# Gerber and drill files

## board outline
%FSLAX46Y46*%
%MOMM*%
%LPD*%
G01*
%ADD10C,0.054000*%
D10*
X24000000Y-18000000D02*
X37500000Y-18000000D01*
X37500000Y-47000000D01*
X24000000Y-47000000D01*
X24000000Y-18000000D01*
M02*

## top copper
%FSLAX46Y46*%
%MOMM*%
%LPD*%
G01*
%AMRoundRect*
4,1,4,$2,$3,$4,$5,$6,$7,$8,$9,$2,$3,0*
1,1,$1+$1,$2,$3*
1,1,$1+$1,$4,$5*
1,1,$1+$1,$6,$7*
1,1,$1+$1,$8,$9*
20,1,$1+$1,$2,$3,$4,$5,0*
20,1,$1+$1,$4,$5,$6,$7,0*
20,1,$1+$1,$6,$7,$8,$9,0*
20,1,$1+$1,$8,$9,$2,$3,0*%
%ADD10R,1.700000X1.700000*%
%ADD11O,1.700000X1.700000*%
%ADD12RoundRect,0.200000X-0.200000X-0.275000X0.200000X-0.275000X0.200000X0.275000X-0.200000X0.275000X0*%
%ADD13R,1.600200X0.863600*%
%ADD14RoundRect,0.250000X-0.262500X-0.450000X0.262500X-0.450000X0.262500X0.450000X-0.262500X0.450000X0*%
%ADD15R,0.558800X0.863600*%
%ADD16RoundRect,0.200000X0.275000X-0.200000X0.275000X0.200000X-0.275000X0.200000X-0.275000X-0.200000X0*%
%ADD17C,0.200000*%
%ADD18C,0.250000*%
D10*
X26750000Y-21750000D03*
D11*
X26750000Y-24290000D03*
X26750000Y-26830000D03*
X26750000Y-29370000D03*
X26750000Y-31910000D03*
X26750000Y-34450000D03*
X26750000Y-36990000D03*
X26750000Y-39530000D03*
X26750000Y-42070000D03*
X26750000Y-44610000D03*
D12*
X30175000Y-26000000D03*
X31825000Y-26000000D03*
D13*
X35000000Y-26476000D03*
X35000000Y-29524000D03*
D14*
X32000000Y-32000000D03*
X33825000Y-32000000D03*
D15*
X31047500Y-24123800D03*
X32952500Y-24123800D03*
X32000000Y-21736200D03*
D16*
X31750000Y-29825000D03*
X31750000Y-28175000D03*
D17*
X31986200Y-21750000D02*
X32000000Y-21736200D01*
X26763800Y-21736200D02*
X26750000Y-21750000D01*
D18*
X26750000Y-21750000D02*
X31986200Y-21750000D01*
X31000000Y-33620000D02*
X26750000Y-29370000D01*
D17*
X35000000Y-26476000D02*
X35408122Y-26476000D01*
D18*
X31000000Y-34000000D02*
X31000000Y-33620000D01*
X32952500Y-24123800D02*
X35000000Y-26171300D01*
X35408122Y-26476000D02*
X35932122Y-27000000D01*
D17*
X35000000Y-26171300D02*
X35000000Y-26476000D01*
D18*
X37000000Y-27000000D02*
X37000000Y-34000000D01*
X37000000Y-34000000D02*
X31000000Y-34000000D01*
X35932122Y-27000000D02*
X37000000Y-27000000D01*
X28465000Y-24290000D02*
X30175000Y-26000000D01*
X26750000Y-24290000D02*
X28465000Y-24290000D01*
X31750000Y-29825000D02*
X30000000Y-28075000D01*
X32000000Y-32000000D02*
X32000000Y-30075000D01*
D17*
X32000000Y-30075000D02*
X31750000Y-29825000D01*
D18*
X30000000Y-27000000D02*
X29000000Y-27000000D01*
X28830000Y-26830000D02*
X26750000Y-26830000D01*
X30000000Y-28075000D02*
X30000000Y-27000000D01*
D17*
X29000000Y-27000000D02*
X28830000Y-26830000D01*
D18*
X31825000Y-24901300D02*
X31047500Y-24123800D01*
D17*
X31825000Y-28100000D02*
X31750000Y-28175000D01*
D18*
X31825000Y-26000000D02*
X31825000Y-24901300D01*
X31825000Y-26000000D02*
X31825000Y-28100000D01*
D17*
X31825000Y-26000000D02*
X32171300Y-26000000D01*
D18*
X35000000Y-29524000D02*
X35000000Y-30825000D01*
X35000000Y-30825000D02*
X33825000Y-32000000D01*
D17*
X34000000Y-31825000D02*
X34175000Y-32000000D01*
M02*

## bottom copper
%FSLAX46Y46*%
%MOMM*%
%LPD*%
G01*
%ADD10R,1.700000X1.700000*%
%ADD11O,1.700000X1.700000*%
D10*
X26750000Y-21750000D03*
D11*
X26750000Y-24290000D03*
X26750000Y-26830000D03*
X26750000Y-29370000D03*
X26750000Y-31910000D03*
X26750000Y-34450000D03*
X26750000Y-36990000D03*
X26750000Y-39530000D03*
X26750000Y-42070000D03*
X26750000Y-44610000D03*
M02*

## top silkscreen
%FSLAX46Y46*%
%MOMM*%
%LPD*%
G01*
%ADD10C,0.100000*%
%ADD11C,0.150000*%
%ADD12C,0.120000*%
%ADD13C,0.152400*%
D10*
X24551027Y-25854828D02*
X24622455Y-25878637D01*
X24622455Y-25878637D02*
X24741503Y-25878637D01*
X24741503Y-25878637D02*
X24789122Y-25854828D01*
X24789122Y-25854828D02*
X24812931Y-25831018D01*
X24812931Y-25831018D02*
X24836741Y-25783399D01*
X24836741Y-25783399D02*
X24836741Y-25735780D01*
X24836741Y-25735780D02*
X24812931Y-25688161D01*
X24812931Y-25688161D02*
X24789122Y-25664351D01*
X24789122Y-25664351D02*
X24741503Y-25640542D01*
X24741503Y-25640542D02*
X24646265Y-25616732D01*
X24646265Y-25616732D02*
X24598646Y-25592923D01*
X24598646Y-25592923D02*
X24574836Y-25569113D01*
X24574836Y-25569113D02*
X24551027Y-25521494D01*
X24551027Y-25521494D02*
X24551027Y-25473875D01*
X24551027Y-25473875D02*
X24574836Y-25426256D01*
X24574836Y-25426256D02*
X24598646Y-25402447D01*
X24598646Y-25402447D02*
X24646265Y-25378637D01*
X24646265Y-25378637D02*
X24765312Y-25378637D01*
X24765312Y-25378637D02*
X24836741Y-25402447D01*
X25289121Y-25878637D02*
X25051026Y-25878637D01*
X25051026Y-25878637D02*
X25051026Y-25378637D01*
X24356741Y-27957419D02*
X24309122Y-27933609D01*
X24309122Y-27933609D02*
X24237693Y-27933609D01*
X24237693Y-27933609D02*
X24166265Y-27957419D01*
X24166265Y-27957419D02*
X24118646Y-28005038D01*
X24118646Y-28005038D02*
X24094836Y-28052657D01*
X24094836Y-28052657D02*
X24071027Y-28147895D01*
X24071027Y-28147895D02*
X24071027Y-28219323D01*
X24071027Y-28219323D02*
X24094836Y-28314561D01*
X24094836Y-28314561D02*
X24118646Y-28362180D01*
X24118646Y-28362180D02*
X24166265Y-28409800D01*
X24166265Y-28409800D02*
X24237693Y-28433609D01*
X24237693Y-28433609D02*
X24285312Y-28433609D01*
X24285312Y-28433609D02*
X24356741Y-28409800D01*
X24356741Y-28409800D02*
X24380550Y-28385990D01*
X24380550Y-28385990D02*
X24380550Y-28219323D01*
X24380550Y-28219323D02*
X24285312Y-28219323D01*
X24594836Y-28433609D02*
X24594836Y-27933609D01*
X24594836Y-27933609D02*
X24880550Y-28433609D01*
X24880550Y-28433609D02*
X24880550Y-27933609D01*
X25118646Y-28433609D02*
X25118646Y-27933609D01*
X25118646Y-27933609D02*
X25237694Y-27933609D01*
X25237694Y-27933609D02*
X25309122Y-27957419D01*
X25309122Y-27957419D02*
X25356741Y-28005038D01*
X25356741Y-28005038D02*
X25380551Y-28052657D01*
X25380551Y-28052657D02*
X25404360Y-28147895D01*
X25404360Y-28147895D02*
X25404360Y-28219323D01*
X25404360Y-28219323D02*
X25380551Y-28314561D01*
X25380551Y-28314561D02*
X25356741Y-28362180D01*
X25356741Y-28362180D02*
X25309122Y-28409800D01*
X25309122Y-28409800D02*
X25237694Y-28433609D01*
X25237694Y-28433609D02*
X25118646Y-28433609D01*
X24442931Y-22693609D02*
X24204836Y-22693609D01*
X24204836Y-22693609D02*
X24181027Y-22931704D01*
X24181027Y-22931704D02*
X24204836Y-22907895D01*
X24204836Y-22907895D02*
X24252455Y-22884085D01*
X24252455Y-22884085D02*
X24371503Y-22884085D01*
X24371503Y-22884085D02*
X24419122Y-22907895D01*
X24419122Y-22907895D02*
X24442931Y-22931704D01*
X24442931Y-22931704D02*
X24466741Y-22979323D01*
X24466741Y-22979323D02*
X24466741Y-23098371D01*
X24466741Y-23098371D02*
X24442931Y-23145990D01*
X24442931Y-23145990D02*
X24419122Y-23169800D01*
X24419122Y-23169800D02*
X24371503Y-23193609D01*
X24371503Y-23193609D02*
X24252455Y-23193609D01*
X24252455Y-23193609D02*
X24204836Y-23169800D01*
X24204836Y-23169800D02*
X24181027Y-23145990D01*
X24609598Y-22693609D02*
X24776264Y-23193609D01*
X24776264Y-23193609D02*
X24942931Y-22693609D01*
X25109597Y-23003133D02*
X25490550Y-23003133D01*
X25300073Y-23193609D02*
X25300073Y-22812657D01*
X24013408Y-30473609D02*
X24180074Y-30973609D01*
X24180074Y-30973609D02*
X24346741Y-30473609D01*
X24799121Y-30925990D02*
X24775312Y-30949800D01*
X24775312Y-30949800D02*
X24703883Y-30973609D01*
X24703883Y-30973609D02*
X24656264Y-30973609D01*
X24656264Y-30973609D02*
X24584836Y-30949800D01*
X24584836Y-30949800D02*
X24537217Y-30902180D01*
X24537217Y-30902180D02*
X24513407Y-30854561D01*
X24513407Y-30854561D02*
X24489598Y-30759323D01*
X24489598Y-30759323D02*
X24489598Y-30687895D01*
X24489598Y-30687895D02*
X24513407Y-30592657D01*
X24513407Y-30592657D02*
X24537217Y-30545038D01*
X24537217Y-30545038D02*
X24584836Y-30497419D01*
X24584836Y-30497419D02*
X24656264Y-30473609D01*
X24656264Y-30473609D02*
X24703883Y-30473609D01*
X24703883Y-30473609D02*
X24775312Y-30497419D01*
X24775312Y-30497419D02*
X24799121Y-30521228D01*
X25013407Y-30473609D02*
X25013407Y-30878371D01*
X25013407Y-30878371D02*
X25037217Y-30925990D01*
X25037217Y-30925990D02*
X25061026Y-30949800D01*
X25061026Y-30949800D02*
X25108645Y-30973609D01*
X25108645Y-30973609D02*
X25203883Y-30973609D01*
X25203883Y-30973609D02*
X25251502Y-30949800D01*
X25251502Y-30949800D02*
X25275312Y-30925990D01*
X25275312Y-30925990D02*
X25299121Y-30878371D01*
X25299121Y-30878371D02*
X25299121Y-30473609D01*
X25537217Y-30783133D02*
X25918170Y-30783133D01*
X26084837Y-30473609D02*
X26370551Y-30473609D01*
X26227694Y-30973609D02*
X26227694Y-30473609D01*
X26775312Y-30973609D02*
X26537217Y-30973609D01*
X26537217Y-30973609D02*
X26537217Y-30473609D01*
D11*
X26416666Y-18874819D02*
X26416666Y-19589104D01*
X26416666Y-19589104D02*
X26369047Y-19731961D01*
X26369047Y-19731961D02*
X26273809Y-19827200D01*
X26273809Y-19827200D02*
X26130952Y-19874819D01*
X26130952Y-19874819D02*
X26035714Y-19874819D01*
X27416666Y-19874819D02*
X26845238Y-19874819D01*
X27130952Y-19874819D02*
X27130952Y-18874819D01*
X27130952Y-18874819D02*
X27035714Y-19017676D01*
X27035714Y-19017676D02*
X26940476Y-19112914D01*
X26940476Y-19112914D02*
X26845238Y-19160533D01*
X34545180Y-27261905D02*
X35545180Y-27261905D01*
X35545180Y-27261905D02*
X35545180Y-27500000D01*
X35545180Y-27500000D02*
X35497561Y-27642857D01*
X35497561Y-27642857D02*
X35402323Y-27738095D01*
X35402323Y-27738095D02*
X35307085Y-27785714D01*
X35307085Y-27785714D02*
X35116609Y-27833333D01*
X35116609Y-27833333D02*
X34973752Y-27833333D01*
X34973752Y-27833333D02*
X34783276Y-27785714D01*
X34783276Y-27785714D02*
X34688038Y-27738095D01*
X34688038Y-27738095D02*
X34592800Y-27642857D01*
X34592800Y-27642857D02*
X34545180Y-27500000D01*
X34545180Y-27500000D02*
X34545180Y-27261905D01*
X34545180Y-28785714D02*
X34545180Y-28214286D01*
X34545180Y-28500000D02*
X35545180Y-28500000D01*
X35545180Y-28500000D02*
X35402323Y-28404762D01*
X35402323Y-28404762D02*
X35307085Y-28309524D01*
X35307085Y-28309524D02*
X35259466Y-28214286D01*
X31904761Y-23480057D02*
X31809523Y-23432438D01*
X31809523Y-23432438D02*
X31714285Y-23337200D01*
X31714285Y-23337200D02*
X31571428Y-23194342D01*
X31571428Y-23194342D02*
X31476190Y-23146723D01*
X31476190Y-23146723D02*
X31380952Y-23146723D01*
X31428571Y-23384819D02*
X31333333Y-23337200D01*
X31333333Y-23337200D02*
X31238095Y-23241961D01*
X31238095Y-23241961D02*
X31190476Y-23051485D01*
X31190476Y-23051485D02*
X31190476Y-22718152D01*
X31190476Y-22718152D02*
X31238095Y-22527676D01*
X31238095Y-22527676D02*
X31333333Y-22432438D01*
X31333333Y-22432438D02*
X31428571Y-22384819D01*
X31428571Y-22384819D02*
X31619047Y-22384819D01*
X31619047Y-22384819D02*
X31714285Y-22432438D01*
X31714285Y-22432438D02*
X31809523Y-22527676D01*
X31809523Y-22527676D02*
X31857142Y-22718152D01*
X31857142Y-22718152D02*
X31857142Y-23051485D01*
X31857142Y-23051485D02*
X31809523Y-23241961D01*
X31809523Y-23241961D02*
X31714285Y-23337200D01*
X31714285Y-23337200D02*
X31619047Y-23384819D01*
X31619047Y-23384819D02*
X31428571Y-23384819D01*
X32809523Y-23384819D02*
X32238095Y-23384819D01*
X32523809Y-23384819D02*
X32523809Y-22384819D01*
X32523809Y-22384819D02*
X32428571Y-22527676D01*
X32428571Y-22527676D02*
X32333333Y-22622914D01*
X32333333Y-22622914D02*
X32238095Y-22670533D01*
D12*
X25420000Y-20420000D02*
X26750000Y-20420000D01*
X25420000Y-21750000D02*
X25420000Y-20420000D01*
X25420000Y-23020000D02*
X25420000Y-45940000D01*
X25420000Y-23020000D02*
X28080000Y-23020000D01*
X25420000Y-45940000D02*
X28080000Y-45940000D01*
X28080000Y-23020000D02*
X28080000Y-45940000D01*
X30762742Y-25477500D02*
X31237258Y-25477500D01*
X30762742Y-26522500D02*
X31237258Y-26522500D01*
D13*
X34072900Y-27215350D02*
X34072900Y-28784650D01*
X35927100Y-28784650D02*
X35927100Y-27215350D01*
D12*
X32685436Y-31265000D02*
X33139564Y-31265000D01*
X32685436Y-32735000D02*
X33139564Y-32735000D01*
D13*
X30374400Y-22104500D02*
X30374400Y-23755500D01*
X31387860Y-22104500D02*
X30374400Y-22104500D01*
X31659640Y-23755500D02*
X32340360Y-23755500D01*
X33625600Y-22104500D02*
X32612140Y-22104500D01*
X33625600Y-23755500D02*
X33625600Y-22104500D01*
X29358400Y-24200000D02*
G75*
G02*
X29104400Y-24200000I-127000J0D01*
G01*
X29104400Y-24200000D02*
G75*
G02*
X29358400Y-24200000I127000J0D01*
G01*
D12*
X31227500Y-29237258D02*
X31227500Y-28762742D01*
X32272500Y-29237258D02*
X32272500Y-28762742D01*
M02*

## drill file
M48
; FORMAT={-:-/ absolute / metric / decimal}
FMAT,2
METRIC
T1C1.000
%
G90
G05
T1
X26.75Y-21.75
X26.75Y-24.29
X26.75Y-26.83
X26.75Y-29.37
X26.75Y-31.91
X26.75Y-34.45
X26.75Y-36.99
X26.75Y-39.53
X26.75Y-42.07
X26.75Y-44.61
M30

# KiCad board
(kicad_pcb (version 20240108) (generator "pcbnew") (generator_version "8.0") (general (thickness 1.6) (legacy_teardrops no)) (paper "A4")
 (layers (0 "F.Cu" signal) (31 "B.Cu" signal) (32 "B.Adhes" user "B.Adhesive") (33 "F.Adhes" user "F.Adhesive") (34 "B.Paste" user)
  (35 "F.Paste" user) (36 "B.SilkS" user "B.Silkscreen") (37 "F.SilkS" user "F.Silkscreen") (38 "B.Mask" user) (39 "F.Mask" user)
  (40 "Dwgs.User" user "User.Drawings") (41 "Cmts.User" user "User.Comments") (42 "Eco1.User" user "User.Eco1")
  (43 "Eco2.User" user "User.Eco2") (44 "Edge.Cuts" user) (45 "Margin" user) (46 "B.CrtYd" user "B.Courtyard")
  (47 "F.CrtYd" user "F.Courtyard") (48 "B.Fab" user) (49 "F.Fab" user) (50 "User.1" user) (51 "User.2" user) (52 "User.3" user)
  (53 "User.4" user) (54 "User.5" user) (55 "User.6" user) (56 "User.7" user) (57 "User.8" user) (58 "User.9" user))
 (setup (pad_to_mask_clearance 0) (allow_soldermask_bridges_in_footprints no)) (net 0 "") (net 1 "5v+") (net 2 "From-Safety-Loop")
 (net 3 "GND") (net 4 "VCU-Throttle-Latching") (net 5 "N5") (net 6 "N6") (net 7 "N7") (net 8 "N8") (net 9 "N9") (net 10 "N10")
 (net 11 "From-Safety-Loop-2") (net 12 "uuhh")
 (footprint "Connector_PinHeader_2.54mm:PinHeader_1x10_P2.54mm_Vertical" (layer "F.Cu") (at 26.75 21.75)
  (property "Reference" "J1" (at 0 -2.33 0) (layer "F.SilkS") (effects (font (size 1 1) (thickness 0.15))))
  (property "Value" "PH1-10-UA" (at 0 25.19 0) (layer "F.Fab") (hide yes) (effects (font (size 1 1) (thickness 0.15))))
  (fp_line (start -1.33 -1.33) (end 0 -1.33) (stroke (width 0.12) (type solid)) (layer "F.SilkS"))
  (fp_line (start -1.33 0) (end -1.33 -1.33) (stroke (width 0.12) (type solid)) (layer "F.SilkS"))
  (fp_line (start -1.33 1.27) (end -1.33 24.19) (stroke (width 0.12) (type solid)) (layer "F.SilkS"))
  (fp_line (start -1.33 1.27) (end 1.33 1.27) (stroke (width 0.12) (type solid)) (layer "F.SilkS"))
  (fp_line (start -1.33 24.19) (end 1.33 24.19) (stroke (width 0.12) (type solid)) (layer "F.SilkS"))
  (fp_line (start 1.33 1.27) (end 1.33 24.19) (stroke (width 0.12) (type solid)) (layer "F.SilkS"))
  (pad "1" thru_hole rect (at 0 0) (size 1.7 1.7) (drill 1) (layers "*.Cu" "*.Mask") (remove_unused_layers no) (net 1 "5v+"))
  (pad "2" thru_hole oval (at 0 2.54) (size 1.7 1.7) (drill 1) (layers "*.Cu" "*.Mask") (remove_unused_layers no) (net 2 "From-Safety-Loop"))
  (pad "3" thru_hole oval (at 0 5.08) (size 1.7 1.7) (drill 1) (layers "*.Cu" "*.Mask") (remove_unused_layers no) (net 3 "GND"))
  (pad "4" thru_hole oval (at 0 7.62) (size 1.7 1.7) (drill 1) (layers "*.Cu" "*.Mask") (remove_unused_layers no)
   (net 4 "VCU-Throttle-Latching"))
  (pad "5" thru_hole oval (at 0 10.16) (size 1.7 1.7) (drill 1) (layers "*.Cu" "*.Mask") (remove_unused_layers no) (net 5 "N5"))
  (pad "6" thru_hole oval (at 0 12.7) (size 1.7 1.7) (drill 1) (layers "*.Cu" "*.Mask") (remove_unused_layers no) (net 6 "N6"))
  (pad "7" thru_hole oval (at 0 15.24) (size 1.7 1.7) (drill 1) (layers "*.Cu" "*.Mask") (remove_unused_layers no) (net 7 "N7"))
  (pad "8" thru_hole oval (at 0 17.78) (size 1.7 1.7) (drill 1) (layers "*.Cu" "*.Mask") (remove_unused_layers no) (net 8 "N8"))
  (pad "9" thru_hole oval (at 0 20.32) (size 1.7 1.7) (drill 1) (layers "*.Cu" "*.Mask") (remove_unused_layers no) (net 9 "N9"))
  (pad "10" thru_hole oval (at 0 22.86) (size 1.7 1.7) (drill 1) (layers "*.Cu" "*.Mask") (remove_unused_layers no) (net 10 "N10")))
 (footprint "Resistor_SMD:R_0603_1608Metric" (layer "F.Cu") (at 31 26)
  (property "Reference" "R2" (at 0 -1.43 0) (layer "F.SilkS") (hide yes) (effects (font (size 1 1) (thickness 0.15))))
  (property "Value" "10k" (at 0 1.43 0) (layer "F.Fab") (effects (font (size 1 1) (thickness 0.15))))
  (fp_line (start -0.237258 -0.5225) (end 0.237258 -0.5225) (stroke (width 0.12) (type solid)) (layer "F.SilkS"))
  (fp_line (start -0.237258 0.5225) (end 0.237258 0.5225) (stroke (width 0.12) (type solid)) (layer "F.SilkS"))
  (pad "1" smd roundrect (at -0.825 0) (size 0.8 0.95) (layers "F.Cu" "F.Paste" "F.Mask") (roundrect_rratio 0.25) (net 2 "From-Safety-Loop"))
  (pad "2" smd roundrect (at 0.825 0) (size 0.8 0.95) (layers "F.Cu" "F.Paste" "F.Mask") (roundrect_rratio 0.25)
   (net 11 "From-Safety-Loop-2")))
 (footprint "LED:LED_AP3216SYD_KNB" (layer "F.Cu") (at 35 28 -90)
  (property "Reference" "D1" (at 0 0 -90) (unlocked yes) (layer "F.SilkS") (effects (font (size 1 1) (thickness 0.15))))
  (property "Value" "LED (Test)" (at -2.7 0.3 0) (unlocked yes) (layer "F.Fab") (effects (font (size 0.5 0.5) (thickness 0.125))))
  (fp_line (start -0.78465 0.9271) (end 0.78465 0.9271) (stroke (width 0.1524) (type solid)) (layer "F.SilkS"))
  (fp_line (start 0.78465 -0.9271) (end -0.78465 -0.9271) (stroke (width 0.1524) (type solid)) (layer "F.SilkS"))
  (pad "1" smd rect (at -1.524 0 270) (size 0.8636 1.6002) (layers "F.Cu" "F.Paste" "F.Mask") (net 4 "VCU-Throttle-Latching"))
  (pad "2" smd rect (at 1.524 0 270) (size 0.8636 1.6002) (layers "F.Cu" "F.Paste" "F.Mask") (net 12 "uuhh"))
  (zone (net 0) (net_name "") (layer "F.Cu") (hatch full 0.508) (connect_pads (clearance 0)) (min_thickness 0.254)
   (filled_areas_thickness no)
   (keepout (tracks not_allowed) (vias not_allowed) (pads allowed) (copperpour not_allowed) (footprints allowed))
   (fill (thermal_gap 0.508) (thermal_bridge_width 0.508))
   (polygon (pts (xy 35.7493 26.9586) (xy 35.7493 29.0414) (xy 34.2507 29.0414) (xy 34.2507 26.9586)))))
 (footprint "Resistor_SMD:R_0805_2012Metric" (layer "F.Cu") (at 32.9125 32)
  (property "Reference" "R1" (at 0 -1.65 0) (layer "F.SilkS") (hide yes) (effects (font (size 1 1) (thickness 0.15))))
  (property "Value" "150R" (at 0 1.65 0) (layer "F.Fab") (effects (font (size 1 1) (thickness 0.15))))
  (fp_line (start -0.227064 -0.735) (end 0.227064 -0.735) (stroke (width 0.12) (type solid)) (layer "F.SilkS"))
  (fp_line (start -0.227064 0.735) (end 0.227064 0.735) (stroke (width 0.12) (type solid)) (layer "F.SilkS"))
  (pad "1" smd roundrect (at -0.9125 0) (size 1.025 1.4) (layers "F.Cu" "F.Paste" "F.Mask") (roundrect_rratio 0.243902) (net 3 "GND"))
  (pad "2" smd roundrect (at 0.9125 0) (size 1.025 1.4) (layers "F.Cu" "F.Paste" "F.Mask") (roundrect_rratio 0.243902) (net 12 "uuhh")))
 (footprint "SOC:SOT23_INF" (layer "F.Cu") (at 32 22.93)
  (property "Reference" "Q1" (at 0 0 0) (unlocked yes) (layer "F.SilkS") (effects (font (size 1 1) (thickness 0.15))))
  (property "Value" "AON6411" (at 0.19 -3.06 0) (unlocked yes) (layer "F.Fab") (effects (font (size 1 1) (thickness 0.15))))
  (fp_line (start -1.6256 -0.8255) (end -1.6256 0.8255) (stroke (width 0.1524) (type solid)) (layer "F.SilkS"))
  (fp_line (start -0.61214 -0.8255) (end -1.6256 -0.8255) (stroke (width 0.1524) (type solid)) (layer "F.SilkS"))
  (fp_line (start -0.34036 0.8255) (end 0.34036 0.8255) (stroke (width 0.1524) (type solid)) (layer "F.SilkS"))
  (fp_line (start 1.6256 -0.8255) (end 0.61214 -0.8255) (stroke (width 0.1524) (type solid)) (layer "F.SilkS"))
  (fp_line (start 1.6256 0.8255) (end 1.6256 -0.8255) (stroke (width 0.1524) (type solid)) (layer "F.SilkS"))
  (fp_circle (center -2.7686 1.27) (end -2.6416 1.27) (stroke (width 0.1524) (type solid)) (fill none) (layer "F.SilkS"))
  (pad "1" smd rect (at -0.9525 1.1938) (size 0.5588 0.8636) (layers "F.Cu" "F.Paste" "F.Mask") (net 11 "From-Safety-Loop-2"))
  (pad "2" smd rect (at 0.9525 1.1938) (size 0.5588 0.8636) (layers "F.Cu" "F.Paste" "F.Mask") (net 4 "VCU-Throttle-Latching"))
  (pad "3" smd rect (at 0 -1.1938) (size 0.5588 0.8636) (layers "F.Cu" "F.Paste" "F.Mask") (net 1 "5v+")))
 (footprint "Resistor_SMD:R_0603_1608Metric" (layer "F.Cu") (at 31.75 29 90)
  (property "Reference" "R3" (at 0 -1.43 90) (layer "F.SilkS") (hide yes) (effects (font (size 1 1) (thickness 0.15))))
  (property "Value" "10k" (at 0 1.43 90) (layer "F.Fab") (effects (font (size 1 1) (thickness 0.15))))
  (fp_line (start -0.237258 -0.5225) (end 0.237258 -0.5225) (stroke (width 0.12) (type solid)) (layer "F.SilkS"))
  (fp_line (start -0.237258 0.5225) (end 0.237258 0.5225) (stroke (width 0.12) (type solid)) (layer "F.SilkS"))
  (pad "1" smd roundrect (at -0.825 0 90) (size 0.8 0.95) (layers "F.Cu" "F.Paste" "F.Mask") (roundrect_rratio 0.25) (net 3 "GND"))
  (pad "2" smd roundrect (at 0.825 0 90) (size 0.8 0.95) (layers "F.Cu" "F.Paste" "F.Mask") (roundrect_rratio 0.25)
   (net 11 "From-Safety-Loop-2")))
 (gr_rect (start 24 18) (end 37.5 47) (stroke (width 0.054) (type default)) (fill none) (layer "Edge.Cuts"))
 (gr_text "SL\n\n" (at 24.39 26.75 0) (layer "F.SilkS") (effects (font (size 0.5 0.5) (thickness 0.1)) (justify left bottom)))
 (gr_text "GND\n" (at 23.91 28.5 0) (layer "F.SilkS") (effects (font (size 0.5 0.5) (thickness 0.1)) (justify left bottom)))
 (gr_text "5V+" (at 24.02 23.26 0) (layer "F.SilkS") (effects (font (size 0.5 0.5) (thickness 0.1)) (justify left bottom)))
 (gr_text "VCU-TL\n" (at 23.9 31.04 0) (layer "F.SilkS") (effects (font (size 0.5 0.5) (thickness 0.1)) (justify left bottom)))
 (segment (start 31.9862 21.75) (end 32 21.7362) (width 0.2) (layer "F.Cu") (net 1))
 (segment (start 26.7638 21.7362) (end 26.75 21.75) (width 0.2) (layer "F.Cu") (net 1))
 (segment (start 26.75 21.75) (end 31.9862 21.75) (width 0.25) (layer "F.Cu") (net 1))
 (segment (start 31 33.62) (end 26.75 29.37) (width 0.25) (layer "F.Cu") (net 4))
 (segment (start 35 26.476) (end 35.408122 26.476) (width 0.2) (layer "F.Cu") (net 4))
 (segment (start 31 34) (end 31 33.62) (width 0.25) (layer "F.Cu") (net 4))
 (segment (start 32.9525 24.1238) (end 35 26.1713) (width 0.25) (layer "F.Cu") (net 4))
 (segment (start 35.408122 26.476) (end 35.932122 27) (width 0.25) (layer "F.Cu") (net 4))
 (segment (start 35 26.1713) (end 35 26.476) (width 0.2) (layer "F.Cu") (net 4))
 (segment (start 37 27) (end 37 34) (width 0.25) (layer "F.Cu") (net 4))
 (segment (start 37 34) (end 31 34) (width 0.25) (layer "F.Cu") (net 4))
 (segment (start 35.932122 27) (end 37 27) (width 0.25) (layer "F.Cu") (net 4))
 (segment (start 28.465 24.29) (end 30.175 26) (width 0.25) (layer "F.Cu") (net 2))
 (segment (start 26.75 24.29) (end 28.465 24.29) (width 0.25) (layer "F.Cu") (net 2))
 (segment (start 31.75 29.825) (end 30 28.075) (width 0.25) (layer "F.Cu") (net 3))
 (segment (start 32 32) (end 32 30.075) (width 0.25) (layer "F.Cu") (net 3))
 (segment (start 32 30.075) (end 31.75 29.825) (width 0.2) (layer "F.Cu") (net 3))
 (segment (start 30 27) (end 29 27) (width 0.25) (layer "F.Cu") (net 3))
 (segment (start 28.83 26.83) (end 26.75 26.83) (width 0.25) (layer "F.Cu") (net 3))
 (segment (start 30 28.075) (end 30 27) (width 0.25) (layer "F.Cu") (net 3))
 (segment (start 29 27) (end 28.83 26.83) (width 0.2) (layer "F.Cu") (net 3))
 (segment (start 31.825 24.9013) (end 31.0475 24.1238) (width 0.25) (layer "F.Cu") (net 11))
 (segment (start 31.825 28.1) (end 31.75 28.175) (width 0.2) (layer "F.Cu") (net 11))
 (segment (start 31.825 26) (end 31.825 24.9013) (width 0.25) (layer "F.Cu") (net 11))
 (segment (start 31.825 26) (end 31.825 28.1) (width 0.25) (layer "F.Cu") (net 11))
 (segment (start 31.825 26) (end 32.1713 26) (width 0.2) (layer "F.Cu") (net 11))
 (segment (start 35 29.524) (end 35 30.825) (width 0.25) (layer "F.Cu") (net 12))
 (segment (start 35 30.825) (end 33.825 32) (width 0.25) (layer "F.Cu") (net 12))
 (segment (start 34 31.825) (end 34.175 32) (width 0.2) (layer "F.Cu") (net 12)))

